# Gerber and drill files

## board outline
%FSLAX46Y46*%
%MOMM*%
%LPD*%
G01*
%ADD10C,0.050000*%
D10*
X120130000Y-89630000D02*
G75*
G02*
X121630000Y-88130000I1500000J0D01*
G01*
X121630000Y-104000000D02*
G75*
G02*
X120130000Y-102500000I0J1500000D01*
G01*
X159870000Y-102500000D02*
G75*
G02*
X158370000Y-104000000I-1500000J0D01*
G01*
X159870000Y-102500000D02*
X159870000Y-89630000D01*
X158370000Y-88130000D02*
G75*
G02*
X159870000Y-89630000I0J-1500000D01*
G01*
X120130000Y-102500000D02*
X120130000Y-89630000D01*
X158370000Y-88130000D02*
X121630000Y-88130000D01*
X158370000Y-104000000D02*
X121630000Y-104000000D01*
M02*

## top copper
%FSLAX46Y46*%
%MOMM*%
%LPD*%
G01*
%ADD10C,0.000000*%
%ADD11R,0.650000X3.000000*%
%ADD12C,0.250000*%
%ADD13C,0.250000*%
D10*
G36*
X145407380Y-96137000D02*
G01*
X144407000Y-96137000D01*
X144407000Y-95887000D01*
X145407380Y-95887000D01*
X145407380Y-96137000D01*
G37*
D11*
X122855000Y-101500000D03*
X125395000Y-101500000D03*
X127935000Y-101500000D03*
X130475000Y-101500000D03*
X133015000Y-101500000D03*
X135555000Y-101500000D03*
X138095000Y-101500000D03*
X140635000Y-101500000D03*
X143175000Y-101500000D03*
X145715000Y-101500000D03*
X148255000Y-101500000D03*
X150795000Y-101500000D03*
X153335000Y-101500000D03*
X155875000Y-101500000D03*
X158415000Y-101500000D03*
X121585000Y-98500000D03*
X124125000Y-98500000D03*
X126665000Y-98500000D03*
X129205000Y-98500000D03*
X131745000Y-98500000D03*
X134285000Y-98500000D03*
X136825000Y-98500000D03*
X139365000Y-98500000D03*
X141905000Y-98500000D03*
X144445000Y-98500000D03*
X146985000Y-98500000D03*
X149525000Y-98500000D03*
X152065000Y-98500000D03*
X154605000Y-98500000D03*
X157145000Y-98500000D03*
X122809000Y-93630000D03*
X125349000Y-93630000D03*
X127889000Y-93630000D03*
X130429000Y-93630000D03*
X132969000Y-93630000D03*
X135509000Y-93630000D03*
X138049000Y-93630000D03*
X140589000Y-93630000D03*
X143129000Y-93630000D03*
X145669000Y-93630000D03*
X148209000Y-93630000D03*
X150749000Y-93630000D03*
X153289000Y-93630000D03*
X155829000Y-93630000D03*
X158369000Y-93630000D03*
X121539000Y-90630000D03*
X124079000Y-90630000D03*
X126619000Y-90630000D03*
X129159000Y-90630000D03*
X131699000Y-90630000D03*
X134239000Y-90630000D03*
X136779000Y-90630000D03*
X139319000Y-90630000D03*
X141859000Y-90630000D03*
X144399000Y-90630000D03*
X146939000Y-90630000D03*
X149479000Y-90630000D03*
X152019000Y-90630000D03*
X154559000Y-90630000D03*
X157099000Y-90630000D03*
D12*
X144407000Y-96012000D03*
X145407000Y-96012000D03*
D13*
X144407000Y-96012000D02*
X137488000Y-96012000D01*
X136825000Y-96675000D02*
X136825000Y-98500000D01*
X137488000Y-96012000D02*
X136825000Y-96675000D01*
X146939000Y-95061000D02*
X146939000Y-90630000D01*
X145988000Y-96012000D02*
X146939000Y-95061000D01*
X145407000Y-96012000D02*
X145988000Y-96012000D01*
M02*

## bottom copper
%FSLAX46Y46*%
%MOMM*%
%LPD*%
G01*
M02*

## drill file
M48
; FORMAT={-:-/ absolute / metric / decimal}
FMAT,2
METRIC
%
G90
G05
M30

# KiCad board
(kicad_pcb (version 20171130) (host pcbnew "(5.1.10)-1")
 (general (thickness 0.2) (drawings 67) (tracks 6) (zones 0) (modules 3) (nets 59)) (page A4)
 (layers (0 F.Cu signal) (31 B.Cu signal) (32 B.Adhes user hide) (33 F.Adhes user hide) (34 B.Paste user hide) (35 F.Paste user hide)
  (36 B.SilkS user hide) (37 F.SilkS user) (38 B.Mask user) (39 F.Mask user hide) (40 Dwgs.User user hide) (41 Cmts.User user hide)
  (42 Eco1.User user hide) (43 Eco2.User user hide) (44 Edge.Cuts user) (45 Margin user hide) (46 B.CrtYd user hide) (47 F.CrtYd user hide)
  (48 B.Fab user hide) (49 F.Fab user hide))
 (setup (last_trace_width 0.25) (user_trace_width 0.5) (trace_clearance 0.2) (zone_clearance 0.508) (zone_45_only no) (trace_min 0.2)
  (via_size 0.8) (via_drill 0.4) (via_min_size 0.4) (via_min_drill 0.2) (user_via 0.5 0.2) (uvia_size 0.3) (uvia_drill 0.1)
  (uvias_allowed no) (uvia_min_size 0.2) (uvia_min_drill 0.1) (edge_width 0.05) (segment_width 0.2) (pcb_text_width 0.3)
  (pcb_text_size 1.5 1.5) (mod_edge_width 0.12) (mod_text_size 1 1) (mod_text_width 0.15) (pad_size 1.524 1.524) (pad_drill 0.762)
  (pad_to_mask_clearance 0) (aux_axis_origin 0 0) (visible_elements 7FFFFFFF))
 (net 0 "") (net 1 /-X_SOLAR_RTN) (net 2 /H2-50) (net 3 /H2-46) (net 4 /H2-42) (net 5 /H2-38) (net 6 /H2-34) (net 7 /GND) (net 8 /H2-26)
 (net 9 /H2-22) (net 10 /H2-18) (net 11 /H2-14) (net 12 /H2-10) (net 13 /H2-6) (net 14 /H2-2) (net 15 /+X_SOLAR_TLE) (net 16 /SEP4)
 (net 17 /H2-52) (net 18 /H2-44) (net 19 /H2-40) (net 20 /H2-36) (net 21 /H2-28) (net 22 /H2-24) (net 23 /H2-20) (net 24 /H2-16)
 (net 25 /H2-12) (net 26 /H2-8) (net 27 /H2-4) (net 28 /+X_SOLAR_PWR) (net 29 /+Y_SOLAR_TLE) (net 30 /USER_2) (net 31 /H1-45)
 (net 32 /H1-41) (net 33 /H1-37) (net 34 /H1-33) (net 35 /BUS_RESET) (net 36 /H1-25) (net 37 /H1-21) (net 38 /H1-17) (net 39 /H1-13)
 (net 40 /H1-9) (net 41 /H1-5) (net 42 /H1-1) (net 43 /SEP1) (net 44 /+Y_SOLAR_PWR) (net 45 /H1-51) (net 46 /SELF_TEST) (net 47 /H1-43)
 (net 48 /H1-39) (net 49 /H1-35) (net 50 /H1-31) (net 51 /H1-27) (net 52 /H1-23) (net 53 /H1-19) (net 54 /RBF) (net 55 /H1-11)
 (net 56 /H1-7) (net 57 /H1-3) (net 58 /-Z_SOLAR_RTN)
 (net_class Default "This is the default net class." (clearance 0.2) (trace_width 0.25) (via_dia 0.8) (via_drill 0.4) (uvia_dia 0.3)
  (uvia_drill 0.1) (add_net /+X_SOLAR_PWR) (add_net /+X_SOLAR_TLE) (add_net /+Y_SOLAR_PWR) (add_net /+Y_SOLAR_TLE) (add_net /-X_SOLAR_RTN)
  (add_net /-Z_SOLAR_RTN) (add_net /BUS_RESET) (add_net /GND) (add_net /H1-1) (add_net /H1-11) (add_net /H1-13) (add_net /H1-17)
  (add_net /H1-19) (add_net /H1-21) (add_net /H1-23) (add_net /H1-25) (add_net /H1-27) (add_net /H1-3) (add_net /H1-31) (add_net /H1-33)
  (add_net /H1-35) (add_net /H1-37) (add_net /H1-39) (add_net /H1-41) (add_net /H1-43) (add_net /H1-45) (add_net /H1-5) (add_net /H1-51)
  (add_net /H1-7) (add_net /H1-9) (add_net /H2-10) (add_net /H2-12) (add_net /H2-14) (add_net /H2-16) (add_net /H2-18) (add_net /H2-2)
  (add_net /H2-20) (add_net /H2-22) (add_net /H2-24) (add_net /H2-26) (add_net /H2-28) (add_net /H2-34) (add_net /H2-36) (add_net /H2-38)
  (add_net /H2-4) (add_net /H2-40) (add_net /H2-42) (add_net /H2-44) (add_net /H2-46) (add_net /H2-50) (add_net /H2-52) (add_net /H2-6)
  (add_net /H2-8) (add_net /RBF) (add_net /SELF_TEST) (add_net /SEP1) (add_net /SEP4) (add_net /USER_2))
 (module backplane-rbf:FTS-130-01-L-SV (layer F.Cu) (at 140 100 270)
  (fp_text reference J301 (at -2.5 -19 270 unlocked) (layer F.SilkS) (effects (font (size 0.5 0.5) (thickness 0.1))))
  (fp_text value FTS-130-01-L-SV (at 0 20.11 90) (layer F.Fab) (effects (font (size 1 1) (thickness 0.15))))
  (pad 29 smd rect (at 1.5 17.145 270) (size 3 0.65) (layers F.Cu F.Paste F.Mask) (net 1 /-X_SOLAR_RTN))
  (pad 27 smd rect (at 1.5 14.605 270) (size 3 0.65) (layers F.Cu F.Paste F.Mask) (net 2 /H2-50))
  (pad 25 smd rect (at 1.5 12.065 270) (size 3 0.65) (layers F.Cu F.Paste F.Mask) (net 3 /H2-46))
  (pad 23 smd rect (at 1.5 9.525 270) (size 3 0.65) (layers F.Cu F.Paste F.Mask) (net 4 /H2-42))
  (pad 21 smd rect (at 1.5 6.985 270) (size 3 0.65) (layers F.Cu F.Paste F.Mask) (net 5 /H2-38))
  (pad 19 smd rect (at 1.5 4.445 270) (size 3 0.65) (layers F.Cu F.Paste F.Mask) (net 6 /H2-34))
  (pad 17 smd rect (at 1.5 1.905 270) (size 3 0.65) (layers F.Cu F.Paste F.Mask) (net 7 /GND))
  (pad 15 smd rect (at 1.5 -0.635 270) (size 3 0.65) (layers F.Cu F.Paste F.Mask) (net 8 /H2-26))
  (pad 13 smd rect (at 1.5 -3.175 270) (size 3 0.65) (layers F.Cu F.Paste F.Mask) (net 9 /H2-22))
  (pad 11 smd rect (at 1.5 -5.715 270) (size 3 0.65) (layers F.Cu F.Paste F.Mask) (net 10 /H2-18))
  (pad 9 smd rect (at 1.5 -8.255 270) (size 3 0.65) (layers F.Cu F.Paste F.Mask) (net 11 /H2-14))
  (pad 7 smd rect (at 1.5 -10.795 270) (size 3 0.65) (layers F.Cu F.Paste F.Mask) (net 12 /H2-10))
  (pad 5 smd rect (at 1.5 -13.335 270) (size 3 0.65) (layers F.Cu F.Paste F.Mask) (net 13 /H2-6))
  (pad 3 smd rect (at 1.5 -15.875 270) (size 3 0.65) (layers F.Cu F.Paste F.Mask) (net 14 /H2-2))
  (pad 1 smd rect (at 1.5 -18.415 270) (size 3 0.65) (layers F.Cu F.Paste F.Mask) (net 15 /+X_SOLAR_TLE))
  (pad 30 smd rect (at -1.5 18.415 270) (size 3 0.65) (layers F.Cu F.Paste F.Mask) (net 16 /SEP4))
  (pad 28 smd rect (at -1.5 15.875 270) (size 3 0.65) (layers F.Cu F.Paste F.Mask) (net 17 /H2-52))
  (pad 26 smd rect (at -1.5 13.335 270) (size 3 0.65) (layers F.Cu F.Paste F.Mask) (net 7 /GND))
  (pad 24 smd rect (at -1.5 10.795 270) (size 3 0.65) (layers F.Cu F.Paste F.Mask) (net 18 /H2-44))
  (pad 22 smd rect (at -1.5 8.255 270) (size 3 0.65) (layers F.Cu F.Paste F.Mask) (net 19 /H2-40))
  (pad 20 smd rect (at -1.5 5.715 270) (size 3 0.65) (layers F.Cu F.Paste F.Mask) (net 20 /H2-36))
  (pad 18 smd rect (at -1.5 3.175 270) (size 3 0.65) (layers F.Cu F.Paste F.Mask) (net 7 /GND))
  (pad 16 smd rect (at -1.5 0.635 270) (size 3 0.65) (layers F.Cu F.Paste F.Mask) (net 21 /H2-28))
  (pad 14 smd rect (at -1.5 -1.905 270) (size 3 0.65) (layers F.Cu F.Paste F.Mask) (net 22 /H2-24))
  (pad 12 smd rect (at -1.5 -4.445 270) (size 3 0.65) (layers F.Cu F.Paste F.Mask) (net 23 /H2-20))
  (pad 10 smd rect (at -1.5 -6.985 270) (size 3 0.65) (layers F.Cu F.Paste F.Mask) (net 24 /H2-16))
  (pad 8 smd rect (at -1.5 -9.525 270) (size 3 0.65) (layers F.Cu F.Paste F.Mask) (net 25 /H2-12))
  (pad 6 smd rect (at -1.5 -12.065 270) (size 3 0.65) (layers F.Cu F.Paste F.Mask) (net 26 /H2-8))
  (pad 4 smd rect (at -1.5 -14.605 270) (size 3 0.65) (layers F.Cu F.Paste F.Mask) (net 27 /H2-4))
  (pad 2 smd rect (at -1.5 -17.145 270) (size 3 0.65) (layers F.Cu F.Paste F.Mask) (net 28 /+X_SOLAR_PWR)))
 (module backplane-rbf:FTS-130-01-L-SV (layer F.Cu) (at 139.954 92.13 270)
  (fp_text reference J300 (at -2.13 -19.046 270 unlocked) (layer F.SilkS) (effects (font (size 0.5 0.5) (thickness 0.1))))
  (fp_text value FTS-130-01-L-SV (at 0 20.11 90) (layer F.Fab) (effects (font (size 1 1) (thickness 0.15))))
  (pad 29 smd rect (at 1.5 17.145 270) (size 3 0.65) (layers F.Cu F.Paste F.Mask) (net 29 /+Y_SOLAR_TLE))
  (pad 27 smd rect (at 1.5 14.605 270) (size 3 0.65) (layers F.Cu F.Paste F.Mask) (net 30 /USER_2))
  (pad 25 smd rect (at 1.5 12.065 270) (size 3 0.65) (layers F.Cu F.Paste F.Mask) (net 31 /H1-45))
  (pad 23 smd rect (at 1.5 9.525 270) (size 3 0.65) (layers F.Cu F.Paste F.Mask) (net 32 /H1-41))
  (pad 21 smd rect (at 1.5 6.985 270) (size 3 0.65) (layers F.Cu F.Paste F.Mask) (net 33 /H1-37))
  (pad 19 smd rect (at 1.5 4.445 270) (size 3 0.65) (layers F.Cu F.Paste F.Mask) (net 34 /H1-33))
  (pad 17 smd rect (at 1.5 1.905 270) (size 3 0.65) (layers F.Cu F.Paste F.Mask) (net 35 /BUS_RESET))
  (pad 15 smd rect (at 1.5 -0.635 270) (size 3 0.65) (layers F.Cu F.Paste F.Mask) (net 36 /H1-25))
  (pad 13 smd rect (at 1.5 -3.175 270) (size 3 0.65) (layers F.Cu F.Paste F.Mask) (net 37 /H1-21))
  (pad 11 smd rect (at 1.5 -5.715 270) (size 3 0.65) (layers F.Cu F.Paste F.Mask) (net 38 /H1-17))
  (pad 9 smd rect (at 1.5 -8.255 270) (size 3 0.65) (layers F.Cu F.Paste F.Mask) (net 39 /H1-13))
  (pad 7 smd rect (at 1.5 -10.795 270) (size 3 0.65) (layers F.Cu F.Paste F.Mask) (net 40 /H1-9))
  (pad 5 smd rect (at 1.5 -13.335 270) (size 3 0.65) (layers F.Cu F.Paste F.Mask) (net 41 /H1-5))
  (pad 3 smd rect (at 1.5 -15.875 270) (size 3 0.65) (layers F.Cu F.Paste F.Mask) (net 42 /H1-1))
  (pad 1 smd rect (at 1.5 -18.415 270) (size 3 0.65) (layers F.Cu F.Paste F.Mask) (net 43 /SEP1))
  (pad 30 smd rect (at -1.5 18.415 270) (size 3 0.65) (layers F.Cu F.Paste F.Mask) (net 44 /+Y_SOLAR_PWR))
  (pad 28 smd rect (at -1.5 15.875 270) (size 3 0.65) (layers F.Cu F.Paste F.Mask) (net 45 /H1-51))
  (pad 26 smd rect (at -1.5 13.335 270) (size 3 0.65) (layers F.Cu F.Paste F.Mask) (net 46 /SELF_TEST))
  (pad 24 smd rect (at -1.5 10.795 270) (size 3 0.65) (layers F.Cu F.Paste F.Mask) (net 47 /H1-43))
  (pad 22 smd rect (at -1.5 8.255 270) (size 3 0.65) (layers F.Cu F.Paste F.Mask) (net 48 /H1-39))
  (pad 20 smd rect (at -1.5 5.715 270) (size 3 0.65) (layers F.Cu F.Paste F.Mask) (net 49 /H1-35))
  (pad 18 smd rect (at -1.5 3.175 270) (size 3 0.65) (layers F.Cu F.Paste F.Mask) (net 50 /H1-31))
  (pad 16 smd rect (at -1.5 0.635 270) (size 3 0.65) (layers F.Cu F.Paste F.Mask) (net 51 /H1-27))
  (pad 14 smd rect (at -1.5 -1.905 270) (size 3 0.65) (layers F.Cu F.Paste F.Mask) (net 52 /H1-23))
  (pad 12 smd rect (at -1.5 -4.445 270) (size 3 0.65) (layers F.Cu F.Paste F.Mask) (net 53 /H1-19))
  (pad 10 smd rect (at -1.5 -6.985 270) (size 3 0.65) (layers F.Cu F.Paste F.Mask) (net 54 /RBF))
  (pad 8 smd rect (at -1.5 -9.525 270) (size 3 0.65) (layers F.Cu F.Paste F.Mask) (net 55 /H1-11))
  (pad 6 smd rect (at -1.5 -12.065 270) (size 3 0.65) (layers F.Cu F.Paste F.Mask) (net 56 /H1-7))
  (pad 4 smd rect (at -1.5 -14.605 270) (size 3 0.65) (layers F.Cu F.Paste F.Mask) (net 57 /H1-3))
  (pad 2 smd rect (at -1.5 -17.145 270) (size 3 0.65) (layers F.Cu F.Paste F.Mask) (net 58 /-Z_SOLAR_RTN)))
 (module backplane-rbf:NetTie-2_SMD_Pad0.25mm (layer F.Cu) (at 144.907 96.012 180)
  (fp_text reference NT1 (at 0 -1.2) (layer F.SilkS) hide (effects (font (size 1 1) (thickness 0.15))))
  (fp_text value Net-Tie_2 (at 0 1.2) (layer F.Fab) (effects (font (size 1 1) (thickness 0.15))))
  (fp_poly (pts (xy -0.50038 -0.125) (xy 0.5 -0.125) (xy 0.5 0.125) (xy -0.50038 0.125)) (layer F.Cu) (width 0))
  (pad 2 smd circle (at 0.5 0 180) (size 0.25 0.25) (layers F.Cu) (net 7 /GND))
  (pad 1 smd circle (at -0.5 0 180) (size 0.25 0.25) (layers F.Cu) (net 54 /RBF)))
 (gr_arc (start 121.63 89.63) (end 120.13 89.63) (angle 90) (layer Edge.Cuts) (width 0.05))
 (gr_arc (start 121.63 102.5) (end 120.13 102.5) (angle -90) (layer Edge.Cuts) (width 0.05))
 (gr_arc (start 158.37 102.5) (end 159.87 102.5) (angle 90) (layer Edge.Cuts) (width 0.05))
 (gr_line (start 159.87 102.5) (end 159.87 89.63) (layer Edge.Cuts) (width 0.05))
 (gr_arc (start 158.37 89.63) (end 159.87 89.63) (angle -90) (layer Edge.Cuts) (width 0.05))
 (gr_line (start 120.13 102.5) (end 120.13 89.63) (layer Edge.Cuts) (width 0.05))
 (gr_line (start 158.37 88.13) (end 121.63 88.13) (layer Edge.Cuts) (width 0.05))
 (gr_line (start 158.37 104) (end 121.63 104) (layer Edge.Cuts) (width 0.05))
 (segment (start 144.407 96.012) (end 137.488 96.012) (width 0.25) (layer F.Cu) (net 7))
 (segment (start 136.825 96.675) (end 136.825 98.5) (width 0.25) (layer F.Cu) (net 7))
 (segment (start 137.488 96.012) (end 136.825 96.675) (width 0.25) (layer F.Cu) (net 7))
 (segment (start 146.939 95.061) (end 146.939 90.63) (width 0.25) (layer F.Cu) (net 54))
 (segment (start 145.988 96.012) (end 146.939 95.061) (width 0.25) (layer F.Cu) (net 54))
 (segment (start 145.407 96.012) (end 145.988 96.012) (width 0.25) (layer F.Cu) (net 54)))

